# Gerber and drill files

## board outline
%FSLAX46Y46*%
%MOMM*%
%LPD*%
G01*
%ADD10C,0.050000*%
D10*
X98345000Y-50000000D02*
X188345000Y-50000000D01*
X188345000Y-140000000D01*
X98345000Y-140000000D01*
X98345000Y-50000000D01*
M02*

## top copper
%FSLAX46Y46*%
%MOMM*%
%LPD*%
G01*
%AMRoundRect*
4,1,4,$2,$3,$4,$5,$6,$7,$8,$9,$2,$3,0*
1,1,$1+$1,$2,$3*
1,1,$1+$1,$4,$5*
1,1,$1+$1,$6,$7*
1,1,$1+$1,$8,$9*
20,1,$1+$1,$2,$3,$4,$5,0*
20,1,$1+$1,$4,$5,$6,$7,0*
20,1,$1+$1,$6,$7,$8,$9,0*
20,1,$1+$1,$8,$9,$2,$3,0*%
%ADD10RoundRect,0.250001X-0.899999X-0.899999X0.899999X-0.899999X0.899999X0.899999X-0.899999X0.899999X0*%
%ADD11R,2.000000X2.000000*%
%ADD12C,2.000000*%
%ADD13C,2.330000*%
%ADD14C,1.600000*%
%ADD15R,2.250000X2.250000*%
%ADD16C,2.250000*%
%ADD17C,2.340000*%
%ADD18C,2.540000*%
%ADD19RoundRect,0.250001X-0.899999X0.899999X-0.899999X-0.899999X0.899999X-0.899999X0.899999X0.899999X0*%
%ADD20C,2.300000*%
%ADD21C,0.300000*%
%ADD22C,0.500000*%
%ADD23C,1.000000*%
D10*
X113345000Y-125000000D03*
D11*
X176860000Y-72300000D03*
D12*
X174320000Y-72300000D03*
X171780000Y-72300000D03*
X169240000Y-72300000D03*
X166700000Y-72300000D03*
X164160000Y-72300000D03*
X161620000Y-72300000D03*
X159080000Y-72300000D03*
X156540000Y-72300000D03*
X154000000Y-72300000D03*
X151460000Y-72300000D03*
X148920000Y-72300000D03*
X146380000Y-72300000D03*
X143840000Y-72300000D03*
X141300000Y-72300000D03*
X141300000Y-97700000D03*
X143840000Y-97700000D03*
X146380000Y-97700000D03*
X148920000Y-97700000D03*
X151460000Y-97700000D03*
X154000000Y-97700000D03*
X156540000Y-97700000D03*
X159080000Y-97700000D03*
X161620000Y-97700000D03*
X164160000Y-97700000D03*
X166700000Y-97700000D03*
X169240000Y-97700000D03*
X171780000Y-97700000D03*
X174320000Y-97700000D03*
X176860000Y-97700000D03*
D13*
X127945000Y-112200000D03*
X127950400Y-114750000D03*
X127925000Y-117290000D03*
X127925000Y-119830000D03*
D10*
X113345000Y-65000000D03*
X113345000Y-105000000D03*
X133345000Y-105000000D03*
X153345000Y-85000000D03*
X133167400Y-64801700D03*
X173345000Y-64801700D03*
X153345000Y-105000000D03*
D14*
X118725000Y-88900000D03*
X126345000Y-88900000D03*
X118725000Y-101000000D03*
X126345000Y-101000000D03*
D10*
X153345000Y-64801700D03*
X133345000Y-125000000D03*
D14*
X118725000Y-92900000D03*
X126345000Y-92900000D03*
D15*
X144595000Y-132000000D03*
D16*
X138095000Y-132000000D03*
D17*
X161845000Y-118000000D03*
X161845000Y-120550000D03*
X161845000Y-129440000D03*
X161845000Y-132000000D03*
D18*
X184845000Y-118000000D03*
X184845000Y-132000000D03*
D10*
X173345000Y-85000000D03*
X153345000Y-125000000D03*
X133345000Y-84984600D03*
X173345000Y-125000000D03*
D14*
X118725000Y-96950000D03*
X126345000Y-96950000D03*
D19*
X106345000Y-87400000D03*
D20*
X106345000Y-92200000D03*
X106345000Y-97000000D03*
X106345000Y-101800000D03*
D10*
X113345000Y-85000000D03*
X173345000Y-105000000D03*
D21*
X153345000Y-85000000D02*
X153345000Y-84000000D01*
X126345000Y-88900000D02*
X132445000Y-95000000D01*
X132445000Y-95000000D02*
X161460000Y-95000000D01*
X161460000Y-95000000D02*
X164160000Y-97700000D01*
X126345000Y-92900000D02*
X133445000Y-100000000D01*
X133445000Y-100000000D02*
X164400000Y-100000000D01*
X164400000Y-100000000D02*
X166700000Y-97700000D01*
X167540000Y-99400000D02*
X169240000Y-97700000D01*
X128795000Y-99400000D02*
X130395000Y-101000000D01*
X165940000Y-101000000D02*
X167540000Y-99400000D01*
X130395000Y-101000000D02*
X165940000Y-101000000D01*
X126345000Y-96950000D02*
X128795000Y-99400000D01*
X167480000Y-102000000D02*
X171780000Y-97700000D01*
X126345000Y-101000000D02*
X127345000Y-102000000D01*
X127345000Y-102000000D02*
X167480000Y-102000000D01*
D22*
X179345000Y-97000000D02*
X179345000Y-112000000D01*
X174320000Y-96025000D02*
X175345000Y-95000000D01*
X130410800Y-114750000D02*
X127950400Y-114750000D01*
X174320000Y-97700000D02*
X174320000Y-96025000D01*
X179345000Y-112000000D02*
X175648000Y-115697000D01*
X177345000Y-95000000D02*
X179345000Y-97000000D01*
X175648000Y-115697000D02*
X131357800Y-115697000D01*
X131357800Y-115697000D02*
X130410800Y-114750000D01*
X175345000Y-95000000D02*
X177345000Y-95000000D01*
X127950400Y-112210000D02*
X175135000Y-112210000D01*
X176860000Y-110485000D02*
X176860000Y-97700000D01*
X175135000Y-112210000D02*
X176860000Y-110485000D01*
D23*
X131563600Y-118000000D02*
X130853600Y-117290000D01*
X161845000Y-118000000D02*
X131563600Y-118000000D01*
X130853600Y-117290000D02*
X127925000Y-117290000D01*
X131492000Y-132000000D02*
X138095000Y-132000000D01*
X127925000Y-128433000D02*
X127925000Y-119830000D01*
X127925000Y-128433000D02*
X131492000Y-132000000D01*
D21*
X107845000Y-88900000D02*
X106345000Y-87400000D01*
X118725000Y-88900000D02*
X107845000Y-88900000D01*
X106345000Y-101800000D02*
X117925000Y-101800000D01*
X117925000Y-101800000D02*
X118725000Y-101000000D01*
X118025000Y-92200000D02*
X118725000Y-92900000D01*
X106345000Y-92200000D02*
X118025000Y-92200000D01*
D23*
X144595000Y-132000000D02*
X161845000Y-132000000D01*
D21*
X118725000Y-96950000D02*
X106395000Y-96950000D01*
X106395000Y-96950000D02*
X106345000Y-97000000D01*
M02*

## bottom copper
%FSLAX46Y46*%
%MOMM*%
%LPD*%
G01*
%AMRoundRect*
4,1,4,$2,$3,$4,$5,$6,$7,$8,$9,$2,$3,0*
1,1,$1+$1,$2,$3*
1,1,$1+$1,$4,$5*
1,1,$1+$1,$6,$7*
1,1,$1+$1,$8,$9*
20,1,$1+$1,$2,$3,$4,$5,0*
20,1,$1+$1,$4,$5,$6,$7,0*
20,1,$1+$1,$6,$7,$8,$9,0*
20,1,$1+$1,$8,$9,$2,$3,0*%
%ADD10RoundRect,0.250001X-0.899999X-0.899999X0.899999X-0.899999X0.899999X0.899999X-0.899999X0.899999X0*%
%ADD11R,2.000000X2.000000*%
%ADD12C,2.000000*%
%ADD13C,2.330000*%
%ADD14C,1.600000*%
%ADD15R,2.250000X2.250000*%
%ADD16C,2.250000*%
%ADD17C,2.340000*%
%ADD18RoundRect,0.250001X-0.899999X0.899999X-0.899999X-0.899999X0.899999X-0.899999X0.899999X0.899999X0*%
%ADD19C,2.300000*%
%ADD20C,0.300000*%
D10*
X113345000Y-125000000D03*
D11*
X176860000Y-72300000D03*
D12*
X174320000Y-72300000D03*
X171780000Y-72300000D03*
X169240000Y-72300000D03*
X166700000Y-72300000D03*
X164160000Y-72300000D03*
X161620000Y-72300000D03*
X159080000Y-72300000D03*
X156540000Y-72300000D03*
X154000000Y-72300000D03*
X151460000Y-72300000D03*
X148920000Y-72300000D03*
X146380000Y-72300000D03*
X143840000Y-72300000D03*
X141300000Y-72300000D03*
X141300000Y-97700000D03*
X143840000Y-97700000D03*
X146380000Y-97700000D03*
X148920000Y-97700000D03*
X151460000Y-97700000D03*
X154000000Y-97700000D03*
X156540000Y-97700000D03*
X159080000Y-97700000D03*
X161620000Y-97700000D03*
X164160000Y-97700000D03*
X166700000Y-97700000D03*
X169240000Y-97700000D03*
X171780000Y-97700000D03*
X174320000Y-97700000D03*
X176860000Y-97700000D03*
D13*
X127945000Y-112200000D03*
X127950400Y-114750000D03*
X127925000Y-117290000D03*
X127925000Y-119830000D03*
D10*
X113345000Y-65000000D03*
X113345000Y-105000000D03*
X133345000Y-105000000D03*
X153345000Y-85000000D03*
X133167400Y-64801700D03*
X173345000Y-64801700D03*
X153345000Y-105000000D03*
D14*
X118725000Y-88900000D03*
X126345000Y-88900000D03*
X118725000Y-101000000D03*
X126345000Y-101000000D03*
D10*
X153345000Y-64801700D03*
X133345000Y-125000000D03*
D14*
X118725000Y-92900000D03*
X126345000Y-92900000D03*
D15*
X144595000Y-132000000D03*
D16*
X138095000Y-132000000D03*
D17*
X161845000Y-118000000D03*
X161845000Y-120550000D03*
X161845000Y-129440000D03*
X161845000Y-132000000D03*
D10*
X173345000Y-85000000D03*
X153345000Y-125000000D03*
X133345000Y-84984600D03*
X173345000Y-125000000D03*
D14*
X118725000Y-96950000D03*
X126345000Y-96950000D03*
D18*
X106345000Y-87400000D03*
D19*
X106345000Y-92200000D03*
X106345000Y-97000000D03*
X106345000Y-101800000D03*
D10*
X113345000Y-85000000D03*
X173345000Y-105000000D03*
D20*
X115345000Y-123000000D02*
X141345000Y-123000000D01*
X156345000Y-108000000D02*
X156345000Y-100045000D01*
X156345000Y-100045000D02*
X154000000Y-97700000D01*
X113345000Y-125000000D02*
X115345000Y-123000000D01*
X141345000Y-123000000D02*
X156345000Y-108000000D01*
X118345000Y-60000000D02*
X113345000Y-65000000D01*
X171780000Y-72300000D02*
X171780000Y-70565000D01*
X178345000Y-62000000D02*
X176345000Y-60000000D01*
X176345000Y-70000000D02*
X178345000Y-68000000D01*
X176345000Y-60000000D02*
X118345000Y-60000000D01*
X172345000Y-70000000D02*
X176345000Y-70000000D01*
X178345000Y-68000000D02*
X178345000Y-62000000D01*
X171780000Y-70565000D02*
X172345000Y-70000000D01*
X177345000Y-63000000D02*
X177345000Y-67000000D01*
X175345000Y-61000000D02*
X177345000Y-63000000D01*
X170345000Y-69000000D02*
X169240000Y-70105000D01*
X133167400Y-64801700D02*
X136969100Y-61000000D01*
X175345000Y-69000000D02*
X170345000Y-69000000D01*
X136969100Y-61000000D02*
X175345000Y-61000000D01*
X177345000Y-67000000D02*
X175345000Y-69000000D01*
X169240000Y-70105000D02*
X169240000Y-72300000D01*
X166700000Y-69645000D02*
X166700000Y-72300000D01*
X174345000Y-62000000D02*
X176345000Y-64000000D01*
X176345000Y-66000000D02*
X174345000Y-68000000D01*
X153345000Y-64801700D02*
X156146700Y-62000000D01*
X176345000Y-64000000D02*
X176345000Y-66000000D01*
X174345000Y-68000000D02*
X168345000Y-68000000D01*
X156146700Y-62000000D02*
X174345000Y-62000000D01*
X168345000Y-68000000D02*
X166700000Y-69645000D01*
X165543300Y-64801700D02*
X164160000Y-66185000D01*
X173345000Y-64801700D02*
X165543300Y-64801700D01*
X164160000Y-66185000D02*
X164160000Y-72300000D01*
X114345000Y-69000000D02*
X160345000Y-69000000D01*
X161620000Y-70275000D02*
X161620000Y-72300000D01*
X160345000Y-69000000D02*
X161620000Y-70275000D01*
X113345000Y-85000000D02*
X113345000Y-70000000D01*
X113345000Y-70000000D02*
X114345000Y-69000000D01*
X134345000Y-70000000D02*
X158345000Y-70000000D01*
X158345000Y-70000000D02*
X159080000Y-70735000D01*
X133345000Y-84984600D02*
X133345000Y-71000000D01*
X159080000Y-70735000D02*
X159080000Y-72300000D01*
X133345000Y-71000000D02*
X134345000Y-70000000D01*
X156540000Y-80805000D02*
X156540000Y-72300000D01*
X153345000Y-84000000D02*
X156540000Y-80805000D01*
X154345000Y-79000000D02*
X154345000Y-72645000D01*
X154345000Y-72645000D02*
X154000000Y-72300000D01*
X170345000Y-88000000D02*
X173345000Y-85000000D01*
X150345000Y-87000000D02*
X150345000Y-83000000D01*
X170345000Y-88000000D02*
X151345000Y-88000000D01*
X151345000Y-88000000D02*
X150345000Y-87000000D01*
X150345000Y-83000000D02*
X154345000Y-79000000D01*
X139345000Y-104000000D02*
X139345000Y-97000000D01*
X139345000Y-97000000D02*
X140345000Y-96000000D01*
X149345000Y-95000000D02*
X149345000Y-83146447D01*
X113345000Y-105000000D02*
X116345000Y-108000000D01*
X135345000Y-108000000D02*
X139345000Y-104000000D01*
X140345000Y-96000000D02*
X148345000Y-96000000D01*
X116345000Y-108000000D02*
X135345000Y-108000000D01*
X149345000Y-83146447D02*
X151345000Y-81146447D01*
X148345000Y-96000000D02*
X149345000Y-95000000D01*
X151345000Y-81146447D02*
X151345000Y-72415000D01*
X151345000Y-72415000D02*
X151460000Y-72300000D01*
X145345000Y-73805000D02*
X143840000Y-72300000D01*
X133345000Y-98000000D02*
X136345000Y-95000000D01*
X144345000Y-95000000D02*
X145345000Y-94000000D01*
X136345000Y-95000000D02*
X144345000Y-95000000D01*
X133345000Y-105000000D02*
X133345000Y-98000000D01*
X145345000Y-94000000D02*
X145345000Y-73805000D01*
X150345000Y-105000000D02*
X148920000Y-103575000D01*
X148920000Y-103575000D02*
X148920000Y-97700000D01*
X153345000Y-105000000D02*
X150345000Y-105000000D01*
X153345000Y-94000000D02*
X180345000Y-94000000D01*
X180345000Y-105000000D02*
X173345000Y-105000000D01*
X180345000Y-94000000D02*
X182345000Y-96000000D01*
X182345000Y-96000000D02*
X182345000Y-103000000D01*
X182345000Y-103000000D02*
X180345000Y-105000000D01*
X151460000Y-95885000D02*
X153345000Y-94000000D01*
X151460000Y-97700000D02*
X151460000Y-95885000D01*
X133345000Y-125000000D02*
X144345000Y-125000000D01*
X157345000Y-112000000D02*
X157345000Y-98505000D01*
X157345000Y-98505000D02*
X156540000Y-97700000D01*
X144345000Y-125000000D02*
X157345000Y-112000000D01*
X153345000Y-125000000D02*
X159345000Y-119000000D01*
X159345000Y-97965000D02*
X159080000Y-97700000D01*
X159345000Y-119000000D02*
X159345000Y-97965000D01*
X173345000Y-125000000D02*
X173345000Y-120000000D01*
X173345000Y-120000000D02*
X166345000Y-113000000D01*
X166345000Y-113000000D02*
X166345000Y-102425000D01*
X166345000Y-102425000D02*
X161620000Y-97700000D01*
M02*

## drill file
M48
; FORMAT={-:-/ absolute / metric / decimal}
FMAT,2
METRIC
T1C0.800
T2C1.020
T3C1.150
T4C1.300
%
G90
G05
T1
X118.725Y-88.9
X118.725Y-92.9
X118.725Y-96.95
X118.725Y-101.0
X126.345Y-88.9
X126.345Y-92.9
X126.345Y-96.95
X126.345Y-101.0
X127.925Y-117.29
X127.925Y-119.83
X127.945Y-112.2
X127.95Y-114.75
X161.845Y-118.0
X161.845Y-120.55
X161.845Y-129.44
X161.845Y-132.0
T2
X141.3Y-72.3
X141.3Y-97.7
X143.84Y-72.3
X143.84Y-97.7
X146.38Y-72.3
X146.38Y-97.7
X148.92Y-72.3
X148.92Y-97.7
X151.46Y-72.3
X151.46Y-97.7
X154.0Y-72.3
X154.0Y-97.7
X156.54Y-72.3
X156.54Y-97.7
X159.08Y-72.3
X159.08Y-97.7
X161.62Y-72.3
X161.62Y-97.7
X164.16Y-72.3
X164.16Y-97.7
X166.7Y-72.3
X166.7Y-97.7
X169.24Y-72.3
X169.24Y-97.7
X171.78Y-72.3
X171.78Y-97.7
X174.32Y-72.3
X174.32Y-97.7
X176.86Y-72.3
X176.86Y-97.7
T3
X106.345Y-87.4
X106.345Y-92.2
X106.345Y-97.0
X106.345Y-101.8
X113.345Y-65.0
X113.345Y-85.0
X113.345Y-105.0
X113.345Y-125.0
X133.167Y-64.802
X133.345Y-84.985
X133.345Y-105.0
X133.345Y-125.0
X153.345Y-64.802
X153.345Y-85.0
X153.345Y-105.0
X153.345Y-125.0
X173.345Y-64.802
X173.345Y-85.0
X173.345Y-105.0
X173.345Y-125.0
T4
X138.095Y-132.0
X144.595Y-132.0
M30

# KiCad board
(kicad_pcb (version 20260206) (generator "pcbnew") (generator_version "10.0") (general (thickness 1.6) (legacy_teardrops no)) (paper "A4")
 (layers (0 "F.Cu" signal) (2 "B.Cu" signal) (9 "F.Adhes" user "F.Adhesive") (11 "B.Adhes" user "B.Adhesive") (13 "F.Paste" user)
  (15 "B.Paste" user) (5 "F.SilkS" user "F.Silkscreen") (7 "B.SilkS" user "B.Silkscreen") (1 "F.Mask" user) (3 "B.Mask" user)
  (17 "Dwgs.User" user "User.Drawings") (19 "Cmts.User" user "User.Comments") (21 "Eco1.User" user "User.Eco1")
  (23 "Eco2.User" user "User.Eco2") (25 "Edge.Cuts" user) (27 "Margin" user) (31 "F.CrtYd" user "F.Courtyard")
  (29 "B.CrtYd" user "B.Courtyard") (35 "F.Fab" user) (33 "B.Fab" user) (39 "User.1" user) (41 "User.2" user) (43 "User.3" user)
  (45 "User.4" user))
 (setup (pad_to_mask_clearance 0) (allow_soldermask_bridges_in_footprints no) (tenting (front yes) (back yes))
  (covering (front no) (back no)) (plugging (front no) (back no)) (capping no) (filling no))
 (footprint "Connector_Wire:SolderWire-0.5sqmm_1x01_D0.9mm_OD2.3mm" (layer "F.Cu") (at 113.345 125)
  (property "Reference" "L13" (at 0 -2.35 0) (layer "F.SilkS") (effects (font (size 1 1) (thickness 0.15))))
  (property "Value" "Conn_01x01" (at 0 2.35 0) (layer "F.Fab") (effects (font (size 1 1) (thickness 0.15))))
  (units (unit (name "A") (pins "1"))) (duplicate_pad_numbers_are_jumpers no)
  (pad "1" thru_hole roundrect (at 0 0) (size 2.3 2.3) (drill 1.15) (layers "*.Cu" "*.Mask") (remove_unused_layers no)
   (roundrect_rratio 0.108696) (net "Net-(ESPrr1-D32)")))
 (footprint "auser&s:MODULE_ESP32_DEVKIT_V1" (layer "F.Cu") (at 161.345 85 -90)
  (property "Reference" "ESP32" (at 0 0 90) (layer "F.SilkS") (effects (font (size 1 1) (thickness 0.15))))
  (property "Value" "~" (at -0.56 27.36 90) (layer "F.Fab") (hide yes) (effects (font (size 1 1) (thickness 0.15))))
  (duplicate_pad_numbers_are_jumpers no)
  (pad "1" thru_hole rect (at -12.7 -15.515 270) (size 2 2) (drill 1.02) (layers "*.Cu" "*.Mask") (remove_unused_layers no)
   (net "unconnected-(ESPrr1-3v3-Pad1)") (solder_mask_margin 0.102))
  (pad "2" thru_hole circle (at -12.7 -12.975 270) (size 2 2) (drill 1.02) (layers "*.Cu" "*.Mask") (remove_unused_layers no)
   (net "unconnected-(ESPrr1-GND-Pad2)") (solder_mask_margin 0.102))
  (pad "3" thru_hole circle (at -12.7 -10.435 270) (size 2 2) (drill 1.02) (layers "*.Cu" "*.Mask") (remove_unused_layers no)
   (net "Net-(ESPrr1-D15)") (solder_mask_margin 0.102))
  (pad "4" thru_hole circle (at -12.7 -7.895 270) (size 2 2) (drill 1.02) (layers "*.Cu" "*.Mask") (remove_unused_layers no)
   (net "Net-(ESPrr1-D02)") (solder_mask_margin 0.102))
  (pad "5" thru_hole circle (at -12.7 -5.355 270) (size 2 2) (drill 1.02) (layers "*.Cu" "*.Mask") (remove_unused_layers no)
   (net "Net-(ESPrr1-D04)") (solder_mask_margin 0.102))
  (pad "6" thru_hole circle (at -12.7 -2.815 270) (size 2 2) (drill 1.02) (layers "*.Cu" "*.Mask") (remove_unused_layers no)
   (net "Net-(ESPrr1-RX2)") (solder_mask_margin 0.102))
  (pad "7" thru_hole circle (at -12.7 -0.275 270) (size 2 2) (drill 1.02) (layers "*.Cu" "*.Mask") (remove_unused_layers no)
   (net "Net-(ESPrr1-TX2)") (solder_mask_margin 0.102))
  (pad "8" thru_hole circle (at -12.7 2.265 270) (size 2 2) (drill 1.02) (layers "*.Cu" "*.Mask") (remove_unused_layers no)
   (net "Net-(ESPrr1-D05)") (solder_mask_margin 0.102))
  (pad "9" thru_hole circle (at -12.7 4.805 270) (size 2 2) (drill 1.02) (layers "*.Cu" "*.Mask") (remove_unused_layers no)
   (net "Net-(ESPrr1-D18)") (solder_mask_margin 0.102))
  (pad "10" thru_hole circle (at -12.7 7.345 270) (size 2 2) (drill 1.02) (layers "*.Cu" "*.Mask") (remove_unused_layers no)
   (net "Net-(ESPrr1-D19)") (solder_mask_margin 0.102))
  (pad "11" thru_hole circle (at -12.7 9.885 270) (size 2 2) (drill 1.02) (layers "*.Cu" "*.Mask") (remove_unused_layers no)
   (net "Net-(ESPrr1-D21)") (solder_mask_margin 0.102))
  (pad "12" thru_hole circle (at -12.7 12.425 270) (size 2 2) (drill 1.02) (layers "*.Cu" "*.Mask") (remove_unused_layers no)
   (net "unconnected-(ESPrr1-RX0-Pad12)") (solder_mask_margin 0.102))
  (pad "13" thru_hole circle (at -12.7 14.965 270) (size 2 2) (drill 1.02) (layers "*.Cu" "*.Mask") (remove_unused_layers no)
   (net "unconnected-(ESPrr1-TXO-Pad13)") (solder_mask_margin 0.102))
  (pad "14" thru_hole circle (at -12.7 17.505 270) (size 2 2) (drill 1.02) (layers "*.Cu" "*.Mask") (remove_unused_layers no)
   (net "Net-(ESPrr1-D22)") (solder_mask_margin 0.102))
  (pad "15" thru_hole circle (at -12.7 20.045 270) (size 2 2) (drill 1.02) (layers "*.Cu" "*.Mask") (remove_unused_layers no)
   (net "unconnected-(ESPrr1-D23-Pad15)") (solder_mask_margin 0.102))
  (pad "16" thru_hole circle (at 12.7 20.045 270) (size 2 2) (drill 1.02) (layers "*.Cu" "*.Mask") (remove_unused_layers no)
   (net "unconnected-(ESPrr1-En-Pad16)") (solder_mask_margin 0.102))
  (pad "17" thru_hole circle (at 12.7 17.505 270) (size 2 2) (drill 1.02) (layers "*.Cu" "*.Mask") (remove_unused_layers no)
   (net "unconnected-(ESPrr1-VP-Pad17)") (solder_mask_margin 0.102))
  (pad "18" thru_hole circle (at 12.7 14.965 270) (size 2 2) (drill 1.02) (layers "*.Cu" "*.Mask") (remove_unused_layers no)
   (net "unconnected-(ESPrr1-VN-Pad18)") (solder_mask_margin 0.102))
  (pad "19" thru_hole circle (at 12.7 12.425 270) (size 2 2) (drill 1.02) (layers "*.Cu" "*.Mask") (remove_unused_layers no)
   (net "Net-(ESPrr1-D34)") (solder_mask_margin 0.102))
  (pad "20" thru_hole circle (at 12.7 9.885 270) (size 2 2) (drill 1.02) (layers "*.Cu" "*.Mask") (remove_unused_layers no)
   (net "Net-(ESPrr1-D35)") (solder_mask_margin 0.102))
  (pad "21" thru_hole circle (at 12.7 7.345 270) (size 2 2) (drill 1.02) (layers "*.Cu" "*.Mask") (remove_unused_layers no)
   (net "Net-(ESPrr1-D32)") (solder_mask_margin 0.102))
  (pad "22" thru_hole circle (at 12.7 4.805 270) (size 2 2) (drill 1.02) (layers "*.Cu" "*.Mask") (remove_unused_layers no)
   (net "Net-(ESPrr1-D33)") (solder_mask_margin 0.102))
  (pad "23" thru_hole circle (at 12.7 2.265 270) (size 2 2) (drill 1.02) (layers "*.Cu" "*.Mask") (remove_unused_layers no)
   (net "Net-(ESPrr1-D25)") (solder_mask_margin 0.102))
  (pad "24" thru_hole circle (at 12.7 -0.275 270) (size 2 2) (drill 1.02) (layers "*.Cu" "*.Mask") (remove_unused_layers no)
   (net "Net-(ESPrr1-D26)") (solder_mask_margin 0.102))
  (pad "25" thru_hole circle (at 12.7 -2.815 270) (size 2 2) (drill 1.02) (layers "*.Cu" "*.Mask") (remove_unused_layers no)
   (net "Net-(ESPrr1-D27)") (solder_mask_margin 0.102))
  (pad "26" thru_hole circle (at 12.7 -5.355 270) (size 2 2) (drill 1.02) (layers "*.Cu" "*.Mask") (remove_unused_layers no)
   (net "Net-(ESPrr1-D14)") (solder_mask_margin 0.102))
  (pad "27" thru_hole circle (at 12.7 -7.895 270) (size 2 2) (drill 1.02) (layers "*.Cu" "*.Mask") (remove_unused_layers no)
   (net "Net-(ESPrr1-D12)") (solder_mask_margin 0.102))
  (pad "28" thru_hole circle (at 12.7 -10.435 270) (size 2 2) (drill 1.02) (layers "*.Cu" "*.Mask") (remove_unused_layers no)
   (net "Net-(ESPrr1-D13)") (solder_mask_margin 0.102))
  (pad "29" thru_hole circle (at 12.7 -12.975 270) (size 2 2) (drill 1.02) (layers "*.Cu" "*.Mask") (remove_unused_layers no)
   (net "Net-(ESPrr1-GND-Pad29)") (solder_mask_margin 0.102))
  (pad "30" thru_hole circle (at 12.7 -15.515 270) (size 2 2) (drill 1.02) (layers "*.Cu" "*.Mask") (remove_unused_layers no)
   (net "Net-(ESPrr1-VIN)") (solder_mask_margin 0.102))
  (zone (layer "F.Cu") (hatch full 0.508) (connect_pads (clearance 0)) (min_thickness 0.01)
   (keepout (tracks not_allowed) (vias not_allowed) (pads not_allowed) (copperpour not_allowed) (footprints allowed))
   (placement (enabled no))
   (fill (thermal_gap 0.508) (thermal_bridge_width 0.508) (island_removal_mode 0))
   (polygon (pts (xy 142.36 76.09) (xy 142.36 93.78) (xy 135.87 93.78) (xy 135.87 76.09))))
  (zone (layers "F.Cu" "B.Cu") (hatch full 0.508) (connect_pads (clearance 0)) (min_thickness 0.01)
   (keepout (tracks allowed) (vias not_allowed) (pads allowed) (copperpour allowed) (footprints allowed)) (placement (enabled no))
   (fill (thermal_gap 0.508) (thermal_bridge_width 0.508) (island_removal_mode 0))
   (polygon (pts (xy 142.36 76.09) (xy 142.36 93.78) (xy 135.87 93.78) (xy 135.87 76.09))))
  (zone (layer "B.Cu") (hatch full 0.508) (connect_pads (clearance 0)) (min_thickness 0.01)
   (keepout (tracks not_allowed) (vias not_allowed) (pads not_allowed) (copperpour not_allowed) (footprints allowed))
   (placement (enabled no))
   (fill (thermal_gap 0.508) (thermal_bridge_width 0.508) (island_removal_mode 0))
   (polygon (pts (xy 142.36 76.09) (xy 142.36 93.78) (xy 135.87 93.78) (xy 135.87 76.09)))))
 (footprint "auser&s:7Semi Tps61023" (layer "F.Cu") (at 123.345 116 -90)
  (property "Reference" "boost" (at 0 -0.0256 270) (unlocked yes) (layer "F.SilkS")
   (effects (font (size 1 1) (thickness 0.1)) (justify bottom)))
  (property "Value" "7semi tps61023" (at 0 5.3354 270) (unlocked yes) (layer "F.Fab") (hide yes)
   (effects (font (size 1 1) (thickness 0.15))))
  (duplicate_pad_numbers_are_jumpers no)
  (pad "1" thru_hole circle (at -3.8 -4.6 270) (size 2.33 2.33) (drill 0.8) (layers "*.Cu" "F.Mask") (remove_unused_layers no)
   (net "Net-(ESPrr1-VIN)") (clearance 0.08))
  (pad "2" thru_hole circle (at -1.25 -4.6054 270) (size 2.33 2.33) (drill 0.8) (layers "*.Cu" "*.Mask") (remove_unused_layers no)
   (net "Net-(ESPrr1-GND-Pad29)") (clearance 0.08))
  (pad "3" thru_hole circle (at 1.29 -4.58 270) (size 2.33 2.33) (drill 0.8) (layers "*.Cu" "*.Mask") (remove_unused_layers no)
   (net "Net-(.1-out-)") (clearance 0.08))
  (pad "4" thru_hole circle (at 3.83 -4.58 270) (size 2.33 2.33) (drill 0.8) (layers "*.Cu" "*.Mask") (remove_unused_layers no)
   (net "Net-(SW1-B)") (clearance 0.08)))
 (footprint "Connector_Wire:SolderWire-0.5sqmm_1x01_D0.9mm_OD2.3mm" (layer "F.Cu") (at 113.345 65)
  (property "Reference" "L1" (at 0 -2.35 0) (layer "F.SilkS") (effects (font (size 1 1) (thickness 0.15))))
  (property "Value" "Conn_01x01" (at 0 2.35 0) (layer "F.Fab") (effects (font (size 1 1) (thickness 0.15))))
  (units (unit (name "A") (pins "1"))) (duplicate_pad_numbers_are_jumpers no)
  (pad "1" thru_hole roundrect (at 0 0) (size 2.3 2.3) (drill 1.15) (layers "*.Cu" "*.Mask") (remove_unused_layers no)
   (roundrect_rratio 0.108696) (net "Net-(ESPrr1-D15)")))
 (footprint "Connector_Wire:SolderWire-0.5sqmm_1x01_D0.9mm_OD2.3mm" (layer "F.Cu") (at 113.345 105)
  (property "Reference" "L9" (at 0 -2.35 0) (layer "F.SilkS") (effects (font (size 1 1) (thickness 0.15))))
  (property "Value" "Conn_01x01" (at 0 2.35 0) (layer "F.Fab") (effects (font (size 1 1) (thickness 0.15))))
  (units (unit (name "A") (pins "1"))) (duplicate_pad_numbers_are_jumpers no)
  (pad "1" thru_hole roundrect (at 0 0) (size 2.3 2.3) (drill 1.15) (layers "*.Cu" "*.Mask") (remove_unused_layers no)
   (roundrect_rratio 0.108696) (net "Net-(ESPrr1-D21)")))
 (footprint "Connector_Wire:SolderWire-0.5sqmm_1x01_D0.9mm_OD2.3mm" (layer "F.Cu") (at 133.345 105)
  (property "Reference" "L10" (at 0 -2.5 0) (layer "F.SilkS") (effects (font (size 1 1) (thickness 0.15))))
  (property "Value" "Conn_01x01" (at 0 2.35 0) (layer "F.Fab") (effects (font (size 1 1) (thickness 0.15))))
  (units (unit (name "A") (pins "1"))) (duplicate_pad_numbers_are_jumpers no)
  (pad "1" thru_hole roundrect (at 0 0) (size 2.3 2.3) (drill 1.15) (layers "*.Cu" "*.Mask") (remove_unused_layers no)
   (roundrect_rratio 0.108696) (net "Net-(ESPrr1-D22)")))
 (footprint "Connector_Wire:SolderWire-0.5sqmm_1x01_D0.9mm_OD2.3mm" (layer "F.Cu") (at 153.345 85)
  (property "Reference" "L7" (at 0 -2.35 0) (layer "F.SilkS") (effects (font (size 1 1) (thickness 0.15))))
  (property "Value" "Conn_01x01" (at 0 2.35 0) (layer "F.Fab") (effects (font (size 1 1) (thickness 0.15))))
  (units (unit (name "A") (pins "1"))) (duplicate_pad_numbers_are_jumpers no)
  (pad "1" thru_hole roundrect (at 0 0) (size 2.3 2.3) (drill 1.15) (layers "*.Cu" "*.Mask") (remove_unused_layers no)
   (roundrect_rratio 0.108696) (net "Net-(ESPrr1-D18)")))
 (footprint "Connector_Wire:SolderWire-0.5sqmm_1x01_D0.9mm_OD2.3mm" (layer "F.Cu") (at 133.1674 64.8017)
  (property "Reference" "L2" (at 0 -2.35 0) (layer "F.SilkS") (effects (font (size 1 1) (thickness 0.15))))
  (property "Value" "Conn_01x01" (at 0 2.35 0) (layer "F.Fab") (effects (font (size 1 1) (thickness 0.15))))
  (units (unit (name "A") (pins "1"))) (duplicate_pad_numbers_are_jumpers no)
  (pad "1" thru_hole roundrect (at 0 0) (size 2.3 2.3) (drill 1.15) (layers "*.Cu" "*.Mask") (remove_unused_layers no)
   (roundrect_rratio 0.108696) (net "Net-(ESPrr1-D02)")))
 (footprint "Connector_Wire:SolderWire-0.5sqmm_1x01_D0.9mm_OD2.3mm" (layer "F.Cu") (at 173.345 64.8017)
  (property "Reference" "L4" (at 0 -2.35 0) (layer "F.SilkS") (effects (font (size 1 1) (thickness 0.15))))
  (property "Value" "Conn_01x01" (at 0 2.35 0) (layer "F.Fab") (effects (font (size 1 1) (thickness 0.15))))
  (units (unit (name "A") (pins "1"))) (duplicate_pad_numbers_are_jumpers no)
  (pad "1" thru_hole roundrect (at 0 0) (size 2.3 2.3) (drill 1.15) (layers "*.Cu" "*.Mask") (remove_unused_layers no)
   (roundrect_rratio 0.108696) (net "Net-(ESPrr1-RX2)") (zone_connect 2)))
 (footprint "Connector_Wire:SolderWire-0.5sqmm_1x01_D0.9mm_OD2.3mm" (layer "F.Cu") (at 153.345 105)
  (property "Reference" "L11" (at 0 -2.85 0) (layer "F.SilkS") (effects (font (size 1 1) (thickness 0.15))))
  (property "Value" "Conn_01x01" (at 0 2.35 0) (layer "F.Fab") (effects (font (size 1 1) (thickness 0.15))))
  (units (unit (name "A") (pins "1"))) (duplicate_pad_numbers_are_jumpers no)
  (pad "1" thru_hole roundrect (at 0 0) (size 2.3 2.3) (drill 1.15) (layers "*.Cu" "*.Mask") (remove_unused_layers no)
   (roundrect_rratio 0.108696) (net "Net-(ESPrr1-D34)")))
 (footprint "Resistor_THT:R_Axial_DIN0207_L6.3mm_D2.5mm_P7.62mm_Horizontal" (layer "F.Cu") (at 118.725 88.9)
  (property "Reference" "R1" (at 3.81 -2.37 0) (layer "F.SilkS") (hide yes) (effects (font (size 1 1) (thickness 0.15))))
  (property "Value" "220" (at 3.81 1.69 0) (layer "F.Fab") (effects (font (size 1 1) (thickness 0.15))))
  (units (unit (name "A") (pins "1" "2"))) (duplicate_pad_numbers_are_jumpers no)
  (pad "1" thru_hole circle (at 0 0) (size 1.6 1.6) (drill 0.8) (layers "*.Cu" "*.Mask") (remove_unused_layers no) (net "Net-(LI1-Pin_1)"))
  (pad "2" thru_hole circle (at 7.62 0) (size 1.6 1.6) (drill 0.8) (layers "*.Cu" "*.Mask") (remove_unused_layers no)
   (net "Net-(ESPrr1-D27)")))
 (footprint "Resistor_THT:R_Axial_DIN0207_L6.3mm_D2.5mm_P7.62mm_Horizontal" (layer "F.Cu") (at 118.725 101)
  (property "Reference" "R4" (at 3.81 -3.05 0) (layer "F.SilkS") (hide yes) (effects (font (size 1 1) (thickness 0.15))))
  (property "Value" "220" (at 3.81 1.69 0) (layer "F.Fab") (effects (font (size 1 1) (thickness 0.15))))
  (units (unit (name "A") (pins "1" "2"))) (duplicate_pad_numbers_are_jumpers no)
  (pad "1" thru_hole circle (at 0 0) (size 1.6 1.6) (drill 0.8) (layers "*.Cu" "*.Mask") (remove_unused_layers no) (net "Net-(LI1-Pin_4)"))
  (pad "2" thru_hole circle (at 7.62 0) (size 1.6 1.6) (drill 0.8) (layers "*.Cu" "*.Mask") (remove_unused_layers no)
   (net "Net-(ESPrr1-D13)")))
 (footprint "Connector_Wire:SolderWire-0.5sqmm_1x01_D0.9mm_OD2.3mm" (layer "F.Cu") (at 153.345 64.8017)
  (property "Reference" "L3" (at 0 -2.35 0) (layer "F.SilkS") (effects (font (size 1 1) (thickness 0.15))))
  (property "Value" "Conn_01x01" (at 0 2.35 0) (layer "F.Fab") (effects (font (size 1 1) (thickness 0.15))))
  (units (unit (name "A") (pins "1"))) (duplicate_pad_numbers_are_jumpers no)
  (pad "1" thru_hole roundrect (at 0 0) (size 2.3 2.3) (drill 1.15) (layers "*.Cu" "*.Mask") (remove_unused_layers no)
   (roundrect_rratio 0.108696) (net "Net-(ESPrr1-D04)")))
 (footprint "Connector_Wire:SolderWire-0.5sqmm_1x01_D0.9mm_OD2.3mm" (layer "F.Cu") (at 133.345 125)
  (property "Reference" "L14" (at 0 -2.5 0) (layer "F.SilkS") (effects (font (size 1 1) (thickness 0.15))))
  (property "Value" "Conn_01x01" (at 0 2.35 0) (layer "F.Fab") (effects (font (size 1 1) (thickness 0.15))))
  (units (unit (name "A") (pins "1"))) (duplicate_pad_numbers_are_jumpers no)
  (pad "1" thru_hole roundrect (at 0 0) (size 2.3 2.3) (drill 1.15) (layers "*.Cu" "*.Mask") (remove_unused_layers no)
   (roundrect_rratio 0.108696) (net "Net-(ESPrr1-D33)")))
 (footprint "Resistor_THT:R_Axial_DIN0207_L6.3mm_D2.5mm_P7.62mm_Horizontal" (layer "F.Cu") (at 118.725 92.9)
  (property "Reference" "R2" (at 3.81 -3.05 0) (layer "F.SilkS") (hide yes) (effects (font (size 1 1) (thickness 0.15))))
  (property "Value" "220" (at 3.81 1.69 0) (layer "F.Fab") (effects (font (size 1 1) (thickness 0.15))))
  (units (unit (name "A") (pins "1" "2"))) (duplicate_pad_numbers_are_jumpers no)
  (pad "1" thru_hole circle (at 0 0) (size 1.6 1.6) (drill 0.8) (layers "*.Cu" "*.Mask") (remove_unused_layers no) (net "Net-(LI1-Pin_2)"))
  (pad "2" thru_hole circle (at 7.62 0) (size 1.6 1.6) (drill 0.8) (layers "*.Cu" "*.Mask") (remove_unused_layers no)
   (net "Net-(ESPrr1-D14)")))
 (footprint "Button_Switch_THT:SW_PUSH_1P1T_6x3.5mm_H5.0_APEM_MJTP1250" (layer "F.Cu") (at 144.595 132 180)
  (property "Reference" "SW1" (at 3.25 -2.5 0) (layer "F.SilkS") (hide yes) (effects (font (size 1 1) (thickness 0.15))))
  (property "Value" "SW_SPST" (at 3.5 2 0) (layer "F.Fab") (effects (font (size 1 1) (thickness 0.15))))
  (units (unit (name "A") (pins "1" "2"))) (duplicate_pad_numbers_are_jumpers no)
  (pad "1" thru_hole rect (at 0 0 270) (size 2.25 2.25) (drill 1.3) (layers "*.Cu" "*.Mask") (remove_unused_layers no) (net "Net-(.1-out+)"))
  (pad "2" thru_hole circle (at 6.5 0 270) (size 2.25 2.25) (drill 1.3) (layers "*.Cu" "*.Mask") (remove_unused_layers no)
   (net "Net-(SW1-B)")))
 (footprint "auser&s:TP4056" (layer "F.Cu") (at 173.345 125 90)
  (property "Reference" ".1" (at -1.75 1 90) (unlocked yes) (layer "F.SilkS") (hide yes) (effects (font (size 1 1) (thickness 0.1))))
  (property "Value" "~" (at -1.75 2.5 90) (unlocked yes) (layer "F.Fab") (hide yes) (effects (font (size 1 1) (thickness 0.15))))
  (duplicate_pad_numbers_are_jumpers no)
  (pad "1" thru_hole circle (at 7 -11.5 90) (size 2.34 2.34) (drill 0.8) (layers "*.Cu" "*.Mask") (remove_unused_layers no)
   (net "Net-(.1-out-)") (clearance 0.08))
  (pad "2" thru_hole circle (at 4.45 -11.5 90) (size 2.34 2.34) (drill 0.8) (layers "*.Cu" "*.Mask") (remove_unused_layers no)
   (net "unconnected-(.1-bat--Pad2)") (clearance 0.08))
  (pad "3" thru_hole circle (at -4.44 -11.5 90) (size 2.34 2.34) (drill 0.8) (layers "*.Cu" "*.Mask") (remove_unused_layers no)
   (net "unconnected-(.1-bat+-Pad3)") (clearance 0.08))
  (pad "4" thru_hole circle (at -7 -11.5 90) (size 2.34 2.34) (drill 0.8) (layers "*.Cu" "*.Mask") (remove_unused_layers no)
   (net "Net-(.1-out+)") (clearance 0.08))
  (pad "5" connect circle (at 7 11.5 90) (size 2.54 2.54) (layers "F.Cu" "F.Mask"))
  (pad "6" connect circle (at -7 11.5 90) (size 2.54 2.54) (layers "F.Cu" "F.Mask")))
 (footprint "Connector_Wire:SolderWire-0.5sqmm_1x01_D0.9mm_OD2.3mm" (layer "F.Cu") (at 173.345 85)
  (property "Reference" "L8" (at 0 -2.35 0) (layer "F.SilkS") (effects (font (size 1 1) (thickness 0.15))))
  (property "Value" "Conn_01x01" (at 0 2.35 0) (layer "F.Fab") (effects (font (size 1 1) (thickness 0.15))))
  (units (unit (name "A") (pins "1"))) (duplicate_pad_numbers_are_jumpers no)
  (pad "1" thru_hole roundrect (at 0 0) (size 2.3 2.3) (drill 1.15) (layers "*.Cu" "*.Mask") (remove_unused_layers no)
   (roundrect_rratio 0.108696) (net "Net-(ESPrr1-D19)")))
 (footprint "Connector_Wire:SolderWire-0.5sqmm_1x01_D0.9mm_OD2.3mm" (layer "F.Cu") (at 153.345 125)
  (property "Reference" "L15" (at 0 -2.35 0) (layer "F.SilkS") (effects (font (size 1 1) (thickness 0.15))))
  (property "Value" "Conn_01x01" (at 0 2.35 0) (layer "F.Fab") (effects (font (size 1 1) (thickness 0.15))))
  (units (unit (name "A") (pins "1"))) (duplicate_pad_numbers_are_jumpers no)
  (pad "1" thru_hole roundrect (at 0 0) (size 2.3 2.3) (drill 1.15) (layers "*.Cu" "*.Mask") (remove_unused_layers no)
   (roundrect_rratio 0.108696) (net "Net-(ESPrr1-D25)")))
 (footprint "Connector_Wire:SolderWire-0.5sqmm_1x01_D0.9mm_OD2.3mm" (layer "F.Cu") (at 133.345 84.9846)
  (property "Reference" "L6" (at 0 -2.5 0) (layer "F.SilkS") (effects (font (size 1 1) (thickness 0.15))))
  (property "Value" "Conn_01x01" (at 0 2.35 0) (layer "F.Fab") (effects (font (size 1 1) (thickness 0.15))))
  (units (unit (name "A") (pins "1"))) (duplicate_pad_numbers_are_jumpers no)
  (pad "1" thru_hole roundrect (at 0 0) (size 2.3 2.3) (drill 1.15) (layers "*.Cu" "*.Mask") (remove_unused_layers no)
   (roundrect_rratio 0.108696) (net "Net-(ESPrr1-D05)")))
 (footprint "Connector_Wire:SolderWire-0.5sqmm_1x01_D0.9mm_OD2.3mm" (layer "F.Cu") (at 173.345 125)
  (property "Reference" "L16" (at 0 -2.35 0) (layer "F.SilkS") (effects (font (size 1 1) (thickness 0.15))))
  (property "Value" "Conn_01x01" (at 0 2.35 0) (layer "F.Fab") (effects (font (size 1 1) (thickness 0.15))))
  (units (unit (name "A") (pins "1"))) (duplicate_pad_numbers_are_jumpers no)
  (pad "1" thru_hole roundrect (at 0 0) (size 2.3 2.3) (drill 1.15) (layers "*.Cu" "*.Mask") (remove_unused_layers no)
   (roundrect_rratio 0.108696) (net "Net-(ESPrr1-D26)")))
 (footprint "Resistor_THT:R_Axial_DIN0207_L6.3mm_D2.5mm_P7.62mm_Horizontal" (layer "F.Cu") (at 118.725 96.95)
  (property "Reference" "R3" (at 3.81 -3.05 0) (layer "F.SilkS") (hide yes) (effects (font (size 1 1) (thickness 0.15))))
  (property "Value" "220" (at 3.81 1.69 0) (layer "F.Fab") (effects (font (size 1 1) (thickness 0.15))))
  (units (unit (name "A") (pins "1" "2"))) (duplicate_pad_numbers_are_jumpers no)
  (pad "1" thru_hole circle (at 0 0) (size 1.6 1.6) (drill 0.8) (layers "*.Cu" "*.Mask") (remove_unused_layers no) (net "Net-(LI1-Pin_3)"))
  (pad "2" thru_hole circle (at 7.62 0) (size 1.6 1.6) (drill 0.8) (layers "*.Cu" "*.Mask") (remove_unused_layers no)
   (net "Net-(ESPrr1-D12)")))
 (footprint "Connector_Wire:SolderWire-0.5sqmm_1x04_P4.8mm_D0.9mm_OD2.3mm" (layer "F.Cu") (at 106.345 87.4 -90)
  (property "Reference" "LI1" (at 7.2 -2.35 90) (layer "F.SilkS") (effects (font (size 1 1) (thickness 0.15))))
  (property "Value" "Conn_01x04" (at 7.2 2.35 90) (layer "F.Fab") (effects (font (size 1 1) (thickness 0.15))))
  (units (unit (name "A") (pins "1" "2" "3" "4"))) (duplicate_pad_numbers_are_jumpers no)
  (pad "1" thru_hole roundrect (at 0 0 270) (size 2.3 2.3) (drill 1.15) (layers "*.Cu" "*.Mask") (remove_unused_layers no)
   (roundrect_rratio 0.108696) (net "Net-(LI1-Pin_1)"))
  (pad "2" thru_hole circle (at 4.8 0 270) (size 2.3 2.3) (drill 1.15) (layers "*.Cu" "*.Mask") (remove_unused_layers no)
   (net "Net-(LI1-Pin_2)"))
  (pad "3" thru_hole circle (at 9.6 0 270) (size 2.3 2.3) (drill 1.15) (layers "*.Cu" "*.Mask") (remove_unused_layers no)
   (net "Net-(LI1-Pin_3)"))
  (pad "4" thru_hole circle (at 14.4 0 270) (size 2.3 2.3) (drill 1.15) (layers "*.Cu" "*.Mask") (remove_unused_layers no)
   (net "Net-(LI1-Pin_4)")))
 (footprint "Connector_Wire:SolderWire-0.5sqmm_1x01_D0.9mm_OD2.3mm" (layer "F.Cu") (at 113.345 85)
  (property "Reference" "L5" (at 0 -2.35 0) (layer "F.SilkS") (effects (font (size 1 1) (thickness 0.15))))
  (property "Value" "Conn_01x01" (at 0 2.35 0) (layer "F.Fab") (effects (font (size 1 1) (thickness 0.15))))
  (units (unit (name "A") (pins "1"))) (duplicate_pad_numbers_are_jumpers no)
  (pad "1" thru_hole roundrect (at 0 0) (size 2.3 2.3) (drill 1.15) (layers "*.Cu" "*.Mask") (remove_unused_layers no)
   (roundrect_rratio 0.108696) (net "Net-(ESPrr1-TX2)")))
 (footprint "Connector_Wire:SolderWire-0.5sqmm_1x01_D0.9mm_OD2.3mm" (layer "F.Cu") (at 173.345 105)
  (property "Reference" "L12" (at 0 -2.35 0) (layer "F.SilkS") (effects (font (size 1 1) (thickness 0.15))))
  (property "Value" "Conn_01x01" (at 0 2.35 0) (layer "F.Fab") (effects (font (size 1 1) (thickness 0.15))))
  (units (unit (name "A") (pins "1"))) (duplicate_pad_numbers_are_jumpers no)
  (pad "1" thru_hole roundrect (at 0 0) (size 2.3 2.3) (drill 1.15) (layers "*.Cu" "*.Mask") (remove_unused_layers no)
   (roundrect_rratio 0.108696) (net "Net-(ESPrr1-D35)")))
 (gr_rect (start 98.345 50) (end 188.345 140) (stroke (width 0.05) (type solid)) (fill no) (layer "Edge.Cuts"))
 (segment (start 115.345 123) (end 141.345 123) (width 0.3) (layer "B.Cu") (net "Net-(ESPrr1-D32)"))
 (segment (start 156.345 108) (end 156.345 100.045) (width 0.3) (layer "B.Cu") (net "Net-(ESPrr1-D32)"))
 (segment (start 156.345 100.045) (end 154 97.7) (width 0.3) (layer "B.Cu") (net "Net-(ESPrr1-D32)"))
 (segment (start 113.345 125) (end 115.345 123) (width 0.3) (layer "B.Cu") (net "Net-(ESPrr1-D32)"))
 (segment (start 141.345 123) (end 156.345 108) (width 0.3) (layer "B.Cu") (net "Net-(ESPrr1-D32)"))
 (segment (start 118.345 60) (end 113.345 65) (width 0.3) (layer "B.Cu") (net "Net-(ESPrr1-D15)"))
 (segment (start 171.78 72.3) (end 171.78 70.565) (width 0.3) (layer "B.Cu") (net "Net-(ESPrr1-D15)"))
 (segment (start 178.345 62) (end 176.345 60) (width 0.3) (layer "B.Cu") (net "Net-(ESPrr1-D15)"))
 (segment (start 176.345 70) (end 178.345 68) (width 0.3) (layer "B.Cu") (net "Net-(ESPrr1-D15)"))
 (segment (start 176.345 60) (end 118.345 60) (width 0.3) (layer "B.Cu") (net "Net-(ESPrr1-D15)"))
 (segment (start 172.345 70) (end 176.345 70) (width 0.3) (layer "B.Cu") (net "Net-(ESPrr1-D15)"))
 (segment (start 178.345 68) (end 178.345 62) (width 0.3) (layer "B.Cu") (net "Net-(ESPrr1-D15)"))
 (segment (start 171.78 70.565) (end 172.345 70) (width 0.3) (layer "B.Cu") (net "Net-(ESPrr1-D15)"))
 (segment (start 177.345 63) (end 177.345 67) (width 0.3) (layer "B.Cu") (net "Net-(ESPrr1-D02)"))
 (segment (start 175.345 61) (end 177.345 63) (width 0.3) (layer "B.Cu") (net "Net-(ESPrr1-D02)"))
 (segment (start 170.345 69) (end 169.24 70.105) (width 0.3) (layer "B.Cu") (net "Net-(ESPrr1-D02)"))
 (segment (start 133.1674 64.8017) (end 136.9691 61) (width 0.3) (layer "B.Cu") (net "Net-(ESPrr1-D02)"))
 (segment (start 175.345 69) (end 170.345 69) (width 0.3) (layer "B.Cu") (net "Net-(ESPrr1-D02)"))
 (segment (start 136.9691 61) (end 175.345 61) (width 0.3) (layer "B.Cu") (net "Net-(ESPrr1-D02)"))
 (segment (start 177.345 67) (end 175.345 69) (width 0.3) (layer "B.Cu") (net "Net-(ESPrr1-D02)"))
 (segment (start 169.24 70.105) (end 169.24 72.3) (width 0.3) (layer "B.Cu") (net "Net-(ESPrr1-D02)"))
 (segment (start 166.7 69.645) (end 166.7 72.3) (width 0.3) (layer "B.Cu") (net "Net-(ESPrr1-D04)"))
 (segment (start 174.345 62) (end 176.345 64) (width 0.3) (layer "B.Cu") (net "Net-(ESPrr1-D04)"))
 (segment (start 176.345 66) (end 174.345 68) (width 0.3) (layer "B.Cu") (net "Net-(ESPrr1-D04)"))
 (segment (start 153.345 64.8017) (end 156.1467 62) (width 0.3) (layer "B.Cu") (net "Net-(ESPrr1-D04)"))
 (segment (start 176.345 64) (end 176.345 66) (width 0.3) (layer "B.Cu") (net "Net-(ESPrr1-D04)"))
 (segment (start 174.345 68) (end 168.345 68) (width 0.3) (layer "B.Cu") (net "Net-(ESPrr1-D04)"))
 (segment (start 156.1467 62) (end 174.345 62) (width 0.3) (layer "B.Cu") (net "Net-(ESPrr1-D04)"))
 (segment (start 168.345 68) (end 166.7 69.645) (width 0.3) (layer "B.Cu") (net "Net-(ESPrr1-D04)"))
 (segment (start 165.5433 64.8017) (end 164.16 66.185) (width 0.3) (layer "B.Cu") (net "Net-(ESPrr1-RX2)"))
 (segment (start 173.345 64.8017) (end 165.5433 64.8017) (width 0.3) (layer "B.Cu") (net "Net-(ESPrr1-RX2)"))
 (segment (start 164.16 66.185) (end 164.16 72.3) (width 0.3) (layer "B.Cu") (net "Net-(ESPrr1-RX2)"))
 (segment (start 114.345 69) (end 160.345 69) (width 0.3) (layer "B.Cu") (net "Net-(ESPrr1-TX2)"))
 (segment (start 161.62 70.275) (end 161.62 72.3) (width 0.3) (layer "B.Cu") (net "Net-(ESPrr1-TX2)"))
 (segment (start 160.345 69) (end 161.62 70.275) (width 0.3) (layer "B.Cu") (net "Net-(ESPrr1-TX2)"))
 (segment (start 113.345 85) (end 113.345 70) (width 0.3) (layer "B.Cu") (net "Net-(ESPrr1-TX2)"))
 (segment (start 113.345 70) (end 114.345 69) (width 0.3) (layer "B.Cu") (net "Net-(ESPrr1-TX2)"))
 (segment (start 134.345 70) (end 158.345 70) (width 0.3) (layer "B.Cu") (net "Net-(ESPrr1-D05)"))
 (segment (start 158.345 70) (end 159.08 70.735) (width 0.3) (layer "B.Cu") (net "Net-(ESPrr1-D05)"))
 (segment (start 133.345 84.9846) (end 133.345 71) (width 0.3) (layer "B.Cu") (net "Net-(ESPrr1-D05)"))
 (segment (start 159.08 70.735) (end 159.08 72.3) (width 0.3) (layer "B.Cu") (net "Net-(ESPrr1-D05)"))
 (segment (start 133.345 71) (end 134.345 70) (width 0.3) (layer "B.Cu") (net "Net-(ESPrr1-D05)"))
 (segment (start 153.345 85) (end 153.345 84) (width 0.3) (layer "F.Cu") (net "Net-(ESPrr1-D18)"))
 (segment (start 156.54 80.805) (end 156.54 72.3) (width 0.3) (layer "B.Cu") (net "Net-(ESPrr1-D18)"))
 (segment (start 153.345 84) (end 156.54 80.805) (width 0.3) (layer "B.Cu") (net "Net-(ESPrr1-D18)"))
 (segment (start 154.345 79) (end 154.345 72.645) (width 0.3) (layer "B.Cu") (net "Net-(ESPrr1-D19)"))
 (segment (start 154.345 72.645) (end 154 72.3) (width 0.3) (layer "B.Cu") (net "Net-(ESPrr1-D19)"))
 (segment (start 170.345 88) (end 173.345 85) (width 0.3) (layer "B.Cu") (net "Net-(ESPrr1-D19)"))
 (segment (start 150.345 87) (end 150.345 83) (width 0.3) (layer "B.Cu") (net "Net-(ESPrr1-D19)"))
 (segment (start 170.345 88) (end 151.345 88) (width 0.3) (layer "B.Cu") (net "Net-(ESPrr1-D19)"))
 (segment (start 151.345 88) (end 150.345 87) (width 0.3) (layer "B.Cu") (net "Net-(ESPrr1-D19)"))
 (segment (start 150.345 83) (end 154.345 79) (width 0.3) (layer "B.Cu") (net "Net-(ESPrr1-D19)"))
 (segment (start 139.345 104) (end 139.345 97) (width 0.3) (layer "B.Cu") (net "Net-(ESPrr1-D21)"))
 (segment (start 139.345 97) (end 140.345 96) (width 0.3) (layer "B.Cu") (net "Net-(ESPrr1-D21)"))
 (segment (start 149.345 95) (end 149.345 83.146447) (width 0.3) (layer "B.Cu") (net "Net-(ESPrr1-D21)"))
 (segment (start 113.345 105) (end 116.345 108) (width 0.3) (layer "B.Cu") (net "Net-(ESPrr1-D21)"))
 (segment (start 135.345 108) (end 139.345 104) (width 0.3) (layer "B.Cu") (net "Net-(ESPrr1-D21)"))
 (segment (start 140.345 96) (end 148.345 96) (width 0.3) (layer "B.Cu") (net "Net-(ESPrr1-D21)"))
 (segment (start 116.345 108) (end 135.345 108) (width 0.3) (layer "B.Cu") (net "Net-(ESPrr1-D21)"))
 (segment (start 149.345 83.146447) (end 151.345 81.146447) (width 0.3) (layer "B.Cu") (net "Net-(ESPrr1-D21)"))
 (segment (start 148.345 96) (end 149.345 95) (width 0.3) (layer "B.Cu") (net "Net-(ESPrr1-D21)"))
 (segment (start 151.345 81.146447) (end 151.345 72.415) (width 0.3) (layer "B.Cu") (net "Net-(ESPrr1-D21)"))
 (segment (start 151.345 72.415) (end 151.46 72.3) (width 0.3) (layer "B.Cu") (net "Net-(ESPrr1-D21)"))
 (segment (start 145.345 73.805) (end 143.84 72.3) (width 0.3) (layer "B.Cu") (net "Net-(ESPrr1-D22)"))
 (segment (start 133.345 98) (end 136.345 95) (width 0.3) (layer "B.Cu") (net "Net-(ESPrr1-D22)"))
 (segment (start 144.345 95) (end 145.345 94) (width 0.3) (layer "B.Cu") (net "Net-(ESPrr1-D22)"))
 (segment (start 136.345 95) (end 144.345 95) (width 0.3) (layer "B.Cu") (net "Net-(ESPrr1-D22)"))
 (segment (start 133.345 105) (end 133.345 98) (width 0.3) (layer "B.Cu") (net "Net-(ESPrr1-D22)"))
 (segment (start 145.345 94) (end 145.345 73.805) (width 0.3) (layer "B.Cu") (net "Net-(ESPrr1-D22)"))
 (segment (start 150.345 105) (end 148.92 103.575) (width 0.3) (layer "B.Cu") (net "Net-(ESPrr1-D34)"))
 (segment (start 148.92 103.575) (end 148.92 97.7) (width 0.3) (layer "B.Cu") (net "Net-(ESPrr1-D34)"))
 (segment (start 153.345 105) (end 150.345 105) (width 0.3) (layer "B.Cu") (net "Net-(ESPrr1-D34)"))
 (segment (start 153.345 94) (end 180.345 94) (width 0.3) (layer "B.Cu") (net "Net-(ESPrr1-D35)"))
 (segment (start 180.345 105) (end 173.345 105) (width 0.3) (layer "B.Cu") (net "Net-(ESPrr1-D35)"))
 (segment (start 180.345 94) (end 182.345 96) (width 0.3) (layer "B.Cu") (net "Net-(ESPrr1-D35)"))
 (segment (start 182.345 96) (end 182.345 103) (width 0.3) (layer "B.Cu") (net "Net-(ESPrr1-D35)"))
 (segment (start 182.345 103) (end 180.345 105) (width 0.3) (layer "B.Cu") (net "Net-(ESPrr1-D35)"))
 (segment (start 151.46 95.885) (end 153.345 94) (width 0.3) (layer "B.Cu") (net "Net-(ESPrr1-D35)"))
 (segment (start 151.46 97.7) (end 151.46 95.885) (width 0.3) (layer "B.Cu") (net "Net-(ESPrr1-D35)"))
 (segment (start 133.345 125) (end 144.345 125) (width 0.3) (layer "B.Cu") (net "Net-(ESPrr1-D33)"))
 (segment (start 157.345 112) (end 157.345 98.505) (width 0.3) (layer "B.Cu") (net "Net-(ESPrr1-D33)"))
 (segment (start 157.345 98.505) (end 156.54 97.7) (width 0.3) (layer "B.Cu") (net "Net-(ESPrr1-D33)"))
 (segment (start 144.345 125) (end 157.345 112) (width 0.3) (layer "B.Cu") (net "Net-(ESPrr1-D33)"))
 (segment (start 153.345 125) (end 159.345 119) (width 0.3) (layer "B.Cu") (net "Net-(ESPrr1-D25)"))
 (segment (start 159.345 97.965) (end 159.08 97.7) (width 0.3) (layer "B.Cu") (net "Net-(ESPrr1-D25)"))
 (segment (start 159.345 119) (end 159.345 97.965) (width 0.3) (layer "B.Cu") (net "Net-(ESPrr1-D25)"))
 (segment (start 173.345 125) (end 173.345 120) (width 0.3) (layer "B.Cu") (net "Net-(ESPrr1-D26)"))
 (segment (start 173.345 120) (end 166.345 113) (width 0.3) (layer "B.Cu") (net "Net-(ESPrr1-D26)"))
 (segment (start 166.345 113) (end 166.345 102.425) (width 0.3) (layer "B.Cu") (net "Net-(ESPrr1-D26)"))
 (segment (start 166.345 102.425) (end 161.62 97.7) (width 0.3) (layer "B.Cu") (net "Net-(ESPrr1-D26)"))
 (segment (start 126.345 88.9) (end 132.445 95) (width 0.3) (layer "F.Cu") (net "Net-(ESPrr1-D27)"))
 (segment (start 132.445 95) (end 161.46 95) (width 0.3) (layer "F.Cu") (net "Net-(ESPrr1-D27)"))
 (segment (start 161.46 95) (end 164.16 97.7) (width 0.3) (layer "F.Cu") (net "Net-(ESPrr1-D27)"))
 (segment (start 126.345 92.9) (end 133.445 100) (width 0.3) (layer "F.Cu") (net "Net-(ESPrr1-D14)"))
 (segment (start 133.445 100) (end 164.4 100) (width 0.3) (layer "F.Cu") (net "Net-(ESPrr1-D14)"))
 (segment (start 164.4 100) (end 166.7 97.7) (width 0.3) (layer "F.Cu") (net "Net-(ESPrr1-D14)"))
 (segment (start 167.54 99.4) (end 169.24 97.7) (width 0.3) (layer "F.Cu") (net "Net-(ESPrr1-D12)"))
 (segment (start 128.795 99.4) (end 130.395 101) (width 0.3) (layer "F.Cu") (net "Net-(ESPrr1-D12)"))
 (segment (start 165.94 101) (end 167.54 99.4) (width 0.3) (layer "F.Cu") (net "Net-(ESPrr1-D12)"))
 (segment (start 130.395 101) (end 165.94 101) (width 0.3) (layer "F.Cu") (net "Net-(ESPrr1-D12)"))
 (segment (start 126.345 96.95) (end 128.795 99.4) (width 0.3) (layer "F.Cu") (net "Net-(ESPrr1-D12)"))
 (segment (start 167.48 102) (end 171.78 97.7) (width 0.3) (layer "F.Cu") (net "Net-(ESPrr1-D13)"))
 (segment (start 126.345 101) (end 127.345 102) (width 0.3) (layer "F.Cu") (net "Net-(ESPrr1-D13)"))
 (segment (start 127.345 102) (end 167.48 102) (width 0.3) (layer "F.Cu") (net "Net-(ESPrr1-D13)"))
 (segment (start 179.345 97) (end 179.345 112) (width 0.5) (layer "F.Cu") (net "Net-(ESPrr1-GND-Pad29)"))
 (segment (start 174.32 96.025) (end 175.345 95) (width 0.5) (layer "F.Cu") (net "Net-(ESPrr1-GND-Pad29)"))
 (segment (start 130.4108 114.75) (end 127.9504 114.75) (width 0.5) (layer "F.Cu") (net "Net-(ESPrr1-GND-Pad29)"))
 (segment (start 174.32 97.7) (end 174.32 96.025) (width 0.5) (layer "F.Cu") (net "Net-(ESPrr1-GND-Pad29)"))
 (segment (start 179.345 112) (end 175.648 115.697) (width 0.5) (layer "F.Cu") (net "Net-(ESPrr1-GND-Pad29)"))
 (segment (start 177.345 95) (end 179.345 97) (width 0.5) (layer "F.Cu") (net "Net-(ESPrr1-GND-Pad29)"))
 (segment (start 175.648 115.697) (end 131.3578 115.697) (width 0.5) (layer "F.Cu") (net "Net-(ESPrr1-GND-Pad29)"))
 (segment (start 131.3578 115.697) (end 130.4108 114.75) (width 0.5) (layer "F.Cu") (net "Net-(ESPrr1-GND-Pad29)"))
 (segment (start 175.345 95) (end 177.345 95) (width 0.5) (layer "F.Cu") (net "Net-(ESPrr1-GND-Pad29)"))
 (segment (start 127.9504 112.21) (end 175.135 112.21) (width 0.5) (layer "F.Cu") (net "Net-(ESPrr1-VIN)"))
 (segment (start 176.86 110.485) (end 176.86 97.7) (width 0.5) (layer "F.Cu") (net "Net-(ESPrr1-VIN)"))
 (segment (start 175.135 112.21) (end 176.86 110.485) (width 0.5) (layer "F.Cu") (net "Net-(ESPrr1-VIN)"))
 (segment (start 131.5636 118) (end 130.8536 117.29) (width 1) (layer "F.Cu") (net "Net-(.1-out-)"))
 (segment (start 161.845 118) (end 131.5636 118) (width 1) (layer "F.Cu") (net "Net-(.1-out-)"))
 (segment (start 130.8536 117.29) (end 127.925 117.29) (width 1) (layer "F.Cu") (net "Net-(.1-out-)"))
 (segment (start 131.492 132) (end 138.095 132) (width 1) (layer "F.Cu") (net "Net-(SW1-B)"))
 (segment (start 127.925 128.433) (end 127.925 119.83) (width 1) (layer "F.Cu") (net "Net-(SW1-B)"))
 (segment (start 127.925 128.433) (end 131.492 132) (width 1) (layer "F.Cu") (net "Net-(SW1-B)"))
 (segment (start 107.845 88.9) (end 106.345 87.4) (width 0.3) (layer "F.Cu") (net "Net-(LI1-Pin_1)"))
 (segment (start 118.725 88.9) (end 107.845 88.9) (width 0.3) (layer "F.Cu") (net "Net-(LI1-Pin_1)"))
 (segment (start 106.345 101.8) (end 117.925 101.8) (width 0.3) (layer "F.Cu") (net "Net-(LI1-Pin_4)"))
 (segment (start 117.925 101.8) (end 118.725 101) (width 0.3) (layer "F.Cu") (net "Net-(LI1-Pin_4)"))
 (segment (start 118.025 92.2) (end 118.725 92.9) (width 0.3) (layer "F.Cu") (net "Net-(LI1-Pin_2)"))
 (segment (start 106.345 92.2) (end 118.025 92.2) (width 0.3) (layer "F.Cu") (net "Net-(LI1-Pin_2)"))
 (segment (start 144.595 132) (end 161.845 132) (width 1) (layer "F.Cu") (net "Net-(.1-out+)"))
 (segment (start 118.725 96.95) (end 106.395 96.95) (width 0.3) (layer "F.Cu") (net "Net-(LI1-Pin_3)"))
 (segment (start 106.395 96.95) (end 106.345 97) (width 0.3) (layer "F.Cu") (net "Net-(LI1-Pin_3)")))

